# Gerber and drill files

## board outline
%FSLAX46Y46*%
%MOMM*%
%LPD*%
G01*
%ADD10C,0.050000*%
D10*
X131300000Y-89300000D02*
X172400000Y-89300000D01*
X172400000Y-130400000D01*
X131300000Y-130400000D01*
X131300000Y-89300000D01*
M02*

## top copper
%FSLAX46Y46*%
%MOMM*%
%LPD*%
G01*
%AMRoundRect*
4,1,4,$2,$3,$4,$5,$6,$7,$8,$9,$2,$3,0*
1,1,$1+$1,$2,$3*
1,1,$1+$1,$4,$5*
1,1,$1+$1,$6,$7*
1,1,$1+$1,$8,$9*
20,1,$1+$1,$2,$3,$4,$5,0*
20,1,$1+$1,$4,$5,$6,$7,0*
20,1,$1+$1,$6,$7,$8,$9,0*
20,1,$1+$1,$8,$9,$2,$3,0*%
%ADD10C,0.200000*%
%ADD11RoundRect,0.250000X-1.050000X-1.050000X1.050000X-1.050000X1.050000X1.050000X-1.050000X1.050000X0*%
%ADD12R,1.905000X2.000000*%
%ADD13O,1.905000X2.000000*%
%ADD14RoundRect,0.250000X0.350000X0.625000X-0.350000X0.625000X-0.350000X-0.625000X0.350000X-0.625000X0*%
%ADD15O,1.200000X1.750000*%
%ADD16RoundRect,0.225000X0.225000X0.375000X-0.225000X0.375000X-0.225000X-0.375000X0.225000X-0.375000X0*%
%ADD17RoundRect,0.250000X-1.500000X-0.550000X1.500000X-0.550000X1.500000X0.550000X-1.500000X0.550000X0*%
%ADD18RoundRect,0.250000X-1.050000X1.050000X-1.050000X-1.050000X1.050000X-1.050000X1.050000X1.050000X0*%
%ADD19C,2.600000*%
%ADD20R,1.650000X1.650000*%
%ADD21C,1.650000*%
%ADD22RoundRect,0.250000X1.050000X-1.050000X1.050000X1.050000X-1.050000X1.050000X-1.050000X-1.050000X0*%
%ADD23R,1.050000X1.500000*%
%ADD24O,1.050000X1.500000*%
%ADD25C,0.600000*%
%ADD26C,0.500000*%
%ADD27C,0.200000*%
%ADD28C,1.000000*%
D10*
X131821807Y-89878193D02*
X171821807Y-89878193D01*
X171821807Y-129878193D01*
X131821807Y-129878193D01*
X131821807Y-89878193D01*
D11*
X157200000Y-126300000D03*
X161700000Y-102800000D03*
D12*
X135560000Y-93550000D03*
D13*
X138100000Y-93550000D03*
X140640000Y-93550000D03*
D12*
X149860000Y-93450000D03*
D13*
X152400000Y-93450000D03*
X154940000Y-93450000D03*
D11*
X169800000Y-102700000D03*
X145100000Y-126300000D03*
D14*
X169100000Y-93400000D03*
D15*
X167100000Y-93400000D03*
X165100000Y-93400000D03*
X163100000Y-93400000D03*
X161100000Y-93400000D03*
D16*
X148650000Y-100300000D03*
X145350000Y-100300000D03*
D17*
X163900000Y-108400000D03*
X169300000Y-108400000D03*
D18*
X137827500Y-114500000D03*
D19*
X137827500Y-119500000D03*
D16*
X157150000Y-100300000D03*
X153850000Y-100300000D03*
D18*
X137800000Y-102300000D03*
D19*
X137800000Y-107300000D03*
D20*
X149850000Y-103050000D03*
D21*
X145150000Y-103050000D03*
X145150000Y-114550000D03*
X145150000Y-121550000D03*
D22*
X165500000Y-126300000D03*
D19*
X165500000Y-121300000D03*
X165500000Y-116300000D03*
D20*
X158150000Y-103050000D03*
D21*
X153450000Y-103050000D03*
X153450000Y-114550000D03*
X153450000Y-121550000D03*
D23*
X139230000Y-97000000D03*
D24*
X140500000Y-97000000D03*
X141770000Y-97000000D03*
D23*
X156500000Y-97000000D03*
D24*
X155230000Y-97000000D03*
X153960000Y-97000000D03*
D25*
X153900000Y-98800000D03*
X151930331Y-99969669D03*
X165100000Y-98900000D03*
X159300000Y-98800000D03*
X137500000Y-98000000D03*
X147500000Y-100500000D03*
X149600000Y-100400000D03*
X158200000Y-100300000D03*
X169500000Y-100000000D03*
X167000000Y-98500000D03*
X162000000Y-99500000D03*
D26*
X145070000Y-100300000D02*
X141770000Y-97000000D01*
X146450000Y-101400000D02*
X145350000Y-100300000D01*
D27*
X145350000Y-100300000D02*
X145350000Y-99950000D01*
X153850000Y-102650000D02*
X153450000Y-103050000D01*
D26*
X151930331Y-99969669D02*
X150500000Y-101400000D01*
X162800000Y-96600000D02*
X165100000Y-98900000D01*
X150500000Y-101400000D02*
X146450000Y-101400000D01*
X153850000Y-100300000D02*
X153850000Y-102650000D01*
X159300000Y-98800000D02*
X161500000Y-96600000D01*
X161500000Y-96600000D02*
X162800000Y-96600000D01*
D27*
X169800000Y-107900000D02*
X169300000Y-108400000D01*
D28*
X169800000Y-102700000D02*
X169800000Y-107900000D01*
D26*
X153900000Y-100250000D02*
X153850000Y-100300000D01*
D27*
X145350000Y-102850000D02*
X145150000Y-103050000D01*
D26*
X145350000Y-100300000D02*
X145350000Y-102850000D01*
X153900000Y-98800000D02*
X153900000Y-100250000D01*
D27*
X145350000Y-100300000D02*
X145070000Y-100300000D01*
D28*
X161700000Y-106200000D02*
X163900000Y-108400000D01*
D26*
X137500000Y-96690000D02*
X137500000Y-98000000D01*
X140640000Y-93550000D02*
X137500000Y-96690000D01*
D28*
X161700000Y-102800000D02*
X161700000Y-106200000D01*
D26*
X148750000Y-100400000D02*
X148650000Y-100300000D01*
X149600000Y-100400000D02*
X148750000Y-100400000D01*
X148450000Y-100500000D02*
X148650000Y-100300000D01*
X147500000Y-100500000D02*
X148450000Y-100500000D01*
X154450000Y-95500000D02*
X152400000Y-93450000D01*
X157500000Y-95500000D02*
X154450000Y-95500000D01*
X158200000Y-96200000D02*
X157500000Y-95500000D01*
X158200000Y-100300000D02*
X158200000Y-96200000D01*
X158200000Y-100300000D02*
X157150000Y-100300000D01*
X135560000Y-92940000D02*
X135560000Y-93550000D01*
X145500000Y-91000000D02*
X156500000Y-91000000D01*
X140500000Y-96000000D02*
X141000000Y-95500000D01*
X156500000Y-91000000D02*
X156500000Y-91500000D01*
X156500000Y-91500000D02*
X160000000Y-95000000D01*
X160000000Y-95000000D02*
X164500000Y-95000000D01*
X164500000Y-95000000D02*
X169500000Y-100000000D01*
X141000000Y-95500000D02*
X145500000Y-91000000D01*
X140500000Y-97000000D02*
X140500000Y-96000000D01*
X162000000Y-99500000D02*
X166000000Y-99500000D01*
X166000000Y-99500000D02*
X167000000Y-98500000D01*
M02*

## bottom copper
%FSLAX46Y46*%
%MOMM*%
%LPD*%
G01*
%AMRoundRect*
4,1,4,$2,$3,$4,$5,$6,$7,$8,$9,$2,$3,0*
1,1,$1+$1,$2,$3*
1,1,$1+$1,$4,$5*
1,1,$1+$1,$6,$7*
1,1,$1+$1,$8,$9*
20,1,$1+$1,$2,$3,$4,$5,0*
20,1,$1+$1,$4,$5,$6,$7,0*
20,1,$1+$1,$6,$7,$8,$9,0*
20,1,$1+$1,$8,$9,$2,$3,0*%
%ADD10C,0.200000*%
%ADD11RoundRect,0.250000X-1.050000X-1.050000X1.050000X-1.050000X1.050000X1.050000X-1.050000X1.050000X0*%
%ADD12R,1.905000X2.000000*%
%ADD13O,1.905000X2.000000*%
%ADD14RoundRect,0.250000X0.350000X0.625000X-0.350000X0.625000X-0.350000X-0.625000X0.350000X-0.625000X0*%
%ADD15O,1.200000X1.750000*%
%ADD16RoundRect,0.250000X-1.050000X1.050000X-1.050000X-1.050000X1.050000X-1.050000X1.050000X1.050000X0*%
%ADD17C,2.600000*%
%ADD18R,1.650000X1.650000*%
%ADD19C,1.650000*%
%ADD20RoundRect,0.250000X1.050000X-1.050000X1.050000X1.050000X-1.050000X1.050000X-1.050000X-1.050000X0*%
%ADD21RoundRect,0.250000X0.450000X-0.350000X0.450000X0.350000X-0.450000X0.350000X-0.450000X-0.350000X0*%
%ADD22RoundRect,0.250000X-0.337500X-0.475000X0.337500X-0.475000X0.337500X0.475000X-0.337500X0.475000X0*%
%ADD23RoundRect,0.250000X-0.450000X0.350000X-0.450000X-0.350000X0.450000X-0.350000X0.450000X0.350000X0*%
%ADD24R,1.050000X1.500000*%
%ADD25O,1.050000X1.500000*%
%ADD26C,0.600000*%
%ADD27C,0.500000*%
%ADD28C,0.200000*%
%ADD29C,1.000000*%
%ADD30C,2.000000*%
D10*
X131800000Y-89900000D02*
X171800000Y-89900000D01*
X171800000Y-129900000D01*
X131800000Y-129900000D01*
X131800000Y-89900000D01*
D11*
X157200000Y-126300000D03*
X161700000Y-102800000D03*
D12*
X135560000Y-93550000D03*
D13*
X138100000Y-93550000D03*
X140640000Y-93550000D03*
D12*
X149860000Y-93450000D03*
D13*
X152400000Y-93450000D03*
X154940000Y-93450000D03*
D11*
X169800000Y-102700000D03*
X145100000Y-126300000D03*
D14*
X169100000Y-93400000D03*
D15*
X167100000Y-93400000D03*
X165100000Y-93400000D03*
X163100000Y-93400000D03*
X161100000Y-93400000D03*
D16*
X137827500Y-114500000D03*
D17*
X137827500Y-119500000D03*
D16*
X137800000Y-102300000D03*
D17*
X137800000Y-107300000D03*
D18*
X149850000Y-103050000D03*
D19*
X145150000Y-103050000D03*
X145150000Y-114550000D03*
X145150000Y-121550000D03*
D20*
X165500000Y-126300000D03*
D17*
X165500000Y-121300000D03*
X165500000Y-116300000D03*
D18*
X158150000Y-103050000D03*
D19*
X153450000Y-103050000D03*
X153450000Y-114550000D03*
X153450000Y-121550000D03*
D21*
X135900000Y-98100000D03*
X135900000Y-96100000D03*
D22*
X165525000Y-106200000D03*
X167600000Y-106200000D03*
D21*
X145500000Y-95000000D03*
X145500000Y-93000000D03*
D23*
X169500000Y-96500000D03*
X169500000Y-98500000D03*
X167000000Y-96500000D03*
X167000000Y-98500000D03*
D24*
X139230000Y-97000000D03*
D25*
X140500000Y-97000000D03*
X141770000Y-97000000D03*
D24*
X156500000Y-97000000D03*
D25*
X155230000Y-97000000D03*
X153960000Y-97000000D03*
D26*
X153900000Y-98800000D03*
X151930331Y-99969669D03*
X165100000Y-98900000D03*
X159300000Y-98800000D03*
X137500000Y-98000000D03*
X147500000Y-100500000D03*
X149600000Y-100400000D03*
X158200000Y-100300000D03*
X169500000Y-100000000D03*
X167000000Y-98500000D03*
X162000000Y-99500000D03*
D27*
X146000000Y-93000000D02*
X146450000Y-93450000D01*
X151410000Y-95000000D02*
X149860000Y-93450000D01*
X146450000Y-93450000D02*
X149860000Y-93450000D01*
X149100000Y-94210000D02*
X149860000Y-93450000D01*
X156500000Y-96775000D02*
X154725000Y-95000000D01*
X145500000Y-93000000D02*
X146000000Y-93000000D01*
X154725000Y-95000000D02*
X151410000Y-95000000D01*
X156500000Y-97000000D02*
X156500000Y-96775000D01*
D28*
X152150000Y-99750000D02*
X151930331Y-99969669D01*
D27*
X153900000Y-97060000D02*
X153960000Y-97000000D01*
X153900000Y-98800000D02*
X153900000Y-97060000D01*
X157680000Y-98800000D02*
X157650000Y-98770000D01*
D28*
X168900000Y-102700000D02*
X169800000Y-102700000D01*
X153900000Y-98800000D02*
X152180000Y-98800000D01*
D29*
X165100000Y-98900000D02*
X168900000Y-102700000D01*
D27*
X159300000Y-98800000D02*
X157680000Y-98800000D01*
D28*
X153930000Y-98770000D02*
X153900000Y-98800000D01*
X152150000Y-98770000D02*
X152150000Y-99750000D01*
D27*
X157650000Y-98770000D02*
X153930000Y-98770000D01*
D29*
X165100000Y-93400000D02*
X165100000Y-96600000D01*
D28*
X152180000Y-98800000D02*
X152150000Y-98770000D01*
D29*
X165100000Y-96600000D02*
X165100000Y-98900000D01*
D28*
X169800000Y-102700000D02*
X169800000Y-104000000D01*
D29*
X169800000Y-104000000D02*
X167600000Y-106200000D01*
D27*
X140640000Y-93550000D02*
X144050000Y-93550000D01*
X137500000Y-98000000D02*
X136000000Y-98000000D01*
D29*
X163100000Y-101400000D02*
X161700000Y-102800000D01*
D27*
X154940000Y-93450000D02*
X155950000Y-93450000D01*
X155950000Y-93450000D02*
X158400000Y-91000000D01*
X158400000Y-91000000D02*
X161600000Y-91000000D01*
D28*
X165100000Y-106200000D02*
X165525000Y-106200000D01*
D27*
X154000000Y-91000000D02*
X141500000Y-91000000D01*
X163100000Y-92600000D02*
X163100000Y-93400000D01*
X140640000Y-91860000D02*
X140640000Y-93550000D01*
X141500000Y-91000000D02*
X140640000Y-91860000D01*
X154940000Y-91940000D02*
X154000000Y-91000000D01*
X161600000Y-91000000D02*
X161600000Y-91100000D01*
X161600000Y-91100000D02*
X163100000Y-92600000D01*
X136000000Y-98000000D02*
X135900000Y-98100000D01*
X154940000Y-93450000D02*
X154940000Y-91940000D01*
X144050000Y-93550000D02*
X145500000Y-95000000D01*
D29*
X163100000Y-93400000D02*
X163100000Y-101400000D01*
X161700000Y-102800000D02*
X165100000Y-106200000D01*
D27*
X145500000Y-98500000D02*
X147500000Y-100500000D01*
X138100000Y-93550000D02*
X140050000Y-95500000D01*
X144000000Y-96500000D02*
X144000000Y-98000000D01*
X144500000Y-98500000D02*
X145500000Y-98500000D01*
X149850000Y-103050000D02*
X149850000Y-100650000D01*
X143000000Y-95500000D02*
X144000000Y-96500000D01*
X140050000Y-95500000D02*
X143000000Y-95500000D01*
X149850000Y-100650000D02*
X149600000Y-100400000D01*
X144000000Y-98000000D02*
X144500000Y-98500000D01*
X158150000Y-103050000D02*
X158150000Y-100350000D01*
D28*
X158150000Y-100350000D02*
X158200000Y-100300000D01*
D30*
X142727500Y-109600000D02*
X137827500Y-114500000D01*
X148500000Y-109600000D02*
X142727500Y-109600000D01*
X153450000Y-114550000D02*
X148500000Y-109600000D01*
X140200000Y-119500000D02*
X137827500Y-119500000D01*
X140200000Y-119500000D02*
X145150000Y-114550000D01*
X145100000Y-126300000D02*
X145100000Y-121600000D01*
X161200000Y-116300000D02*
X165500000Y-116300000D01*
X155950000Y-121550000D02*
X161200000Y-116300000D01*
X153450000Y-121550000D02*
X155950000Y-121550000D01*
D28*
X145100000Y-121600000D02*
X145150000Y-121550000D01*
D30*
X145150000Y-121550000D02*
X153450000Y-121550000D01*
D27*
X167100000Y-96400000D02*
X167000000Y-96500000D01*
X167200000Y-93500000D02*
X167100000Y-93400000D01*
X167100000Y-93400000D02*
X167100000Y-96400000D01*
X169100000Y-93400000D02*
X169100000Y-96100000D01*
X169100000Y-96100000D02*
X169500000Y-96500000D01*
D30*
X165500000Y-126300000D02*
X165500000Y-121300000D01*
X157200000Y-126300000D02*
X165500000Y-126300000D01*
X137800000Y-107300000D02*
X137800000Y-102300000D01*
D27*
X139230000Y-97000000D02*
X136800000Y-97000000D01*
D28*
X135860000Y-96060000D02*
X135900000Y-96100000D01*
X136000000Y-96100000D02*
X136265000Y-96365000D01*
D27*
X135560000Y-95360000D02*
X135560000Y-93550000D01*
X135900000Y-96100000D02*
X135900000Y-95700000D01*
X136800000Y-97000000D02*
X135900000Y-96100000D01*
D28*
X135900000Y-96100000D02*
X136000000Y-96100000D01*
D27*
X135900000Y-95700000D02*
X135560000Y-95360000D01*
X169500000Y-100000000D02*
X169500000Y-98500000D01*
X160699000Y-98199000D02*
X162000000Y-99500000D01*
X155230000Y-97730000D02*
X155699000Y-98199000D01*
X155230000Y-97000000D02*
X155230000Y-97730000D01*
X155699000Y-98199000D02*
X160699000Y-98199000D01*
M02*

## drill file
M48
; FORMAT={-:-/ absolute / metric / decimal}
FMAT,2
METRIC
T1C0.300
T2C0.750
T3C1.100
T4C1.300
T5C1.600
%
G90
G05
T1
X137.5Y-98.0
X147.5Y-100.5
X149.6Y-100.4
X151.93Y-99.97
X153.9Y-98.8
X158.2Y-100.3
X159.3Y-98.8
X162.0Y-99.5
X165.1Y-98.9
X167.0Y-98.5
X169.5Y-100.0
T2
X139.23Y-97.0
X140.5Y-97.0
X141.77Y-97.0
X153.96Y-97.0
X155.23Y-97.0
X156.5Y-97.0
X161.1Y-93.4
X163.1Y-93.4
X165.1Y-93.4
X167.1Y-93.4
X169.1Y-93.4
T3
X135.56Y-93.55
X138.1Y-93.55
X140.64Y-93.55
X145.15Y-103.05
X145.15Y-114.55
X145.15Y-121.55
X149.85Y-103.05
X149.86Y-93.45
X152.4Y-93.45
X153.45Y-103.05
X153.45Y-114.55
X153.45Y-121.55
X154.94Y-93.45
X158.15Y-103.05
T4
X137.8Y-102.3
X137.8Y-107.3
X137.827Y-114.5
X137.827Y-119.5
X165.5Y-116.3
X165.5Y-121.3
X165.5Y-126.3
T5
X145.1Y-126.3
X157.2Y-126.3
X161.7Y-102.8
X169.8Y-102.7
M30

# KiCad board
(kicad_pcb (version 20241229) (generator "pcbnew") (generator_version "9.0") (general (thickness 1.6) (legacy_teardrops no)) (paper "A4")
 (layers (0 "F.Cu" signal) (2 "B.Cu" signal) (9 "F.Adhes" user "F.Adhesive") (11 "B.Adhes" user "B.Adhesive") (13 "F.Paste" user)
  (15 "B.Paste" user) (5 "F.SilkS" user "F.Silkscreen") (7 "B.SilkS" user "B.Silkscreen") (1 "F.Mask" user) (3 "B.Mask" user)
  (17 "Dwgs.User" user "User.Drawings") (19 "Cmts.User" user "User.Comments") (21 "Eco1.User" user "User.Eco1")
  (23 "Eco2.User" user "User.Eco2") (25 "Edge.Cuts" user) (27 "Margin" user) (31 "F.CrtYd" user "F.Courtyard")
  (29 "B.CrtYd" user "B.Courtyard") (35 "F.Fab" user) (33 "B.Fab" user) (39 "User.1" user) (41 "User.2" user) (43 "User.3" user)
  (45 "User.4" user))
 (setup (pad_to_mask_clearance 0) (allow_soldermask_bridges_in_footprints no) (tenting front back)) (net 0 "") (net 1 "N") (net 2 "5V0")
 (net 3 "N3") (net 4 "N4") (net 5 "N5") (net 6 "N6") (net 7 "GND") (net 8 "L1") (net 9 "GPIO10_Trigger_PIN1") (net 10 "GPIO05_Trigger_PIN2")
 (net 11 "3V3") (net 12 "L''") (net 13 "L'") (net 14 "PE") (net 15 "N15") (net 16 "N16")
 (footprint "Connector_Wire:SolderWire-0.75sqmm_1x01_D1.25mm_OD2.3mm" (layer "F.Cu") (at 157.2 126.3)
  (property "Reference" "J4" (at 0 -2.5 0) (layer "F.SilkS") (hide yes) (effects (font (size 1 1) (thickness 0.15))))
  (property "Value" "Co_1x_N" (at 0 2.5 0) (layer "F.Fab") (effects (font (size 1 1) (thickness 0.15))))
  (pad "1" thru_hole roundrect (at 0 0) (size 2.6 2.6) (drill 1.6) (layers "*.Cu" "*.Mask") (remove_unused_layers no)
   (roundrect_rratio 0.096154) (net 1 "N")))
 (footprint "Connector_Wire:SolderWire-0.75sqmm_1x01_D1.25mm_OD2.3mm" (layer "F.Cu") (at 161.7 102.8)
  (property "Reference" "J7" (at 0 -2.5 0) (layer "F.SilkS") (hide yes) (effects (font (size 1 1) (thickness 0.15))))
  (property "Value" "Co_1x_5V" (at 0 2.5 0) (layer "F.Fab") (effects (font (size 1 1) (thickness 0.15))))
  (pad "1" thru_hole roundrect (at 0 0) (size 2.6 2.6) (drill 1.6) (layers "*.Cu" "*.Mask") (remove_unused_layers no)
   (roundrect_rratio 0.096154) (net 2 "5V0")))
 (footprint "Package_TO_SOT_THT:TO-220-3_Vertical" (layer "F.Cu") (at 135.56 93.55)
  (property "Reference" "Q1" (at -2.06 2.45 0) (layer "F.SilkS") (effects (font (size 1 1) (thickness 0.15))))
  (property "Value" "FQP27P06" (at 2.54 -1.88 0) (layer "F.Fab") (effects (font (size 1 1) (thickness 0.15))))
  (pad "1" thru_hole rect (at 0 0) (size 1.905 2) (drill 1.1) (layers "*.Cu" "*.Mask") (remove_unused_layers no) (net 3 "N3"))
  (pad "2" thru_hole oval (at 2.54 0) (size 1.905 2) (drill 1.1) (layers "*.Cu" "*.Mask") (remove_unused_layers no) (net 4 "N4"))
  (pad "3" thru_hole oval (at 5.08 0) (size 1.905 2) (drill 1.1) (layers "*.Cu" "*.Mask") (remove_unused_layers no) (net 2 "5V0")))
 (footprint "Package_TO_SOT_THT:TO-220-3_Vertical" (layer "F.Cu") (at 149.86 93.45)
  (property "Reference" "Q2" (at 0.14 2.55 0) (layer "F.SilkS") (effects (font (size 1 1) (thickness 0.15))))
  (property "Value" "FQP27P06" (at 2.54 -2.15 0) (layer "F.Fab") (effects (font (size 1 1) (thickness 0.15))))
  (pad "1" thru_hole rect (at 0 0) (size 1.905 2) (drill 1.1) (layers "*.Cu" "*.Mask") (remove_unused_layers no) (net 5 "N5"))
  (pad "2" thru_hole oval (at 2.54 0) (size 1.905 2) (drill 1.1) (layers "*.Cu" "*.Mask") (remove_unused_layers no) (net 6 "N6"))
  (pad "3" thru_hole oval (at 5.08 0) (size 1.905 2) (drill 1.1) (layers "*.Cu" "*.Mask") (remove_unused_layers no) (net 2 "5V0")))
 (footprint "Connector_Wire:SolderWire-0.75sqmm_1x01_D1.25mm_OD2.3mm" (layer "F.Cu") (at 169.8 102.7)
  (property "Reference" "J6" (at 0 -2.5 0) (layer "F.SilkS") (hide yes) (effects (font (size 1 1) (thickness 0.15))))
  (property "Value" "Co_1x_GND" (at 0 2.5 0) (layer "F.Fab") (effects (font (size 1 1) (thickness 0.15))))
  (pad "1" thru_hole roundrect (at 0 0) (size 2.6 2.6) (drill 1.6) (layers "*.Cu" "*.Mask") (remove_unused_layers no)
   (roundrect_rratio 0.096154) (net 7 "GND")))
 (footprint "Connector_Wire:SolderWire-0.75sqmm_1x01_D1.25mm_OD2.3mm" (layer "F.Cu") (at 145.1 126.3)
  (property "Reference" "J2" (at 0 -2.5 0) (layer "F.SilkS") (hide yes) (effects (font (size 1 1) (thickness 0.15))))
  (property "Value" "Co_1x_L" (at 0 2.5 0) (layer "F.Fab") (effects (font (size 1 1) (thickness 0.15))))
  (pad "1" thru_hole roundrect (at 0 0) (size 2.6 2.6) (drill 1.6) (layers "*.Cu" "*.Mask") (remove_unused_layers no)
   (roundrect_rratio 0.096154) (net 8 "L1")))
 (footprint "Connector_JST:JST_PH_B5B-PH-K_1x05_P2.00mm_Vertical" (layer "F.Cu") (at 169.1 93.4 180)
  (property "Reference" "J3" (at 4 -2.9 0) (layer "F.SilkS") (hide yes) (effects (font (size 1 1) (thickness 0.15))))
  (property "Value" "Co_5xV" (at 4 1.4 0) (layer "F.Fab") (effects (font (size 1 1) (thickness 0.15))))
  (pad "1" thru_hole roundrect (at 0 0 180) (size 1.2 1.75) (drill 0.75) (layers "*.Cu" "*.Mask") (remove_unused_layers no)
   (roundrect_rratio 0.208333) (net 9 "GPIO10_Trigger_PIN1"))
  (pad "2" thru_hole oval (at 2 0 180) (size 1.2 1.75) (drill 0.75) (layers "*.Cu" "*.Mask") (remove_unused_layers no)
   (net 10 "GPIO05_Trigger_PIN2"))
  (pad "3" thru_hole oval (at 4 0 180) (size 1.2 1.75) (drill 0.75) (layers "*.Cu" "*.Mask") (remove_unused_layers no) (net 7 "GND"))
  (pad "4" thru_hole oval (at 6 0 180) (size 1.2 1.75) (drill 0.75) (layers "*.Cu" "*.Mask") (remove_unused_layers no) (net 2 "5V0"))
  (pad "5" thru_hole oval (at 8 0 180) (size 1.2 1.75) (drill 0.75) (layers "*.Cu" "*.Mask") (remove_unused_layers no) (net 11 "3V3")))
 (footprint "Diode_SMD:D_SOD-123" (layer "F.Cu") (at 147 100.3 180)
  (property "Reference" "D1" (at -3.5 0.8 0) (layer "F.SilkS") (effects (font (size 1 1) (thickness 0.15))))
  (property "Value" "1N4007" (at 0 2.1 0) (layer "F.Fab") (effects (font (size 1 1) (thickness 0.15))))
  (pad "1" smd roundrect (at -1.65 0 180) (size 0.9 1.2) (layers "F.Cu" "F.Mask" "F.Paste") (roundrect_rratio 0.25) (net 4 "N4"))
  (pad "2" smd roundrect (at 1.65 0 180) (size 0.9 1.2) (layers "F.Cu" "F.Mask" "F.Paste") (roundrect_rratio 0.25) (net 7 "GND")))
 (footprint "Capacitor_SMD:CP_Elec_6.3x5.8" (layer "F.Cu") (at 166.6 108.4)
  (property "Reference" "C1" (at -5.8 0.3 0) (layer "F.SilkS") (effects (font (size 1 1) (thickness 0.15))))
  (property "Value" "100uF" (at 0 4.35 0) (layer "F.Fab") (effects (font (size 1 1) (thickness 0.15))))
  (pad "1" smd roundrect (at -2.7 0) (size 3.5 1.6) (layers "F.Cu" "F.Mask" "F.Paste") (roundrect_rratio 0.15625) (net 2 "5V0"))
  (pad "2" smd roundrect (at 2.7 0) (size 3.5 1.6) (layers "F.Cu" "F.Mask" "F.Paste") (roundrect_rratio 0.15625) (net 7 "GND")))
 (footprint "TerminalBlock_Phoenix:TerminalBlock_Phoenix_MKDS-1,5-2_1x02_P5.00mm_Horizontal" (layer "F.Cu") (at 137.8275 114.5 -90)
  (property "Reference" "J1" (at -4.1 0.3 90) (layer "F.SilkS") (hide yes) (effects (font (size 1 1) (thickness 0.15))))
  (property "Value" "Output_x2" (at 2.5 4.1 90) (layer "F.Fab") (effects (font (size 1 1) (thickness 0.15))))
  (pad "1" thru_hole roundrect (at 0 0 270) (size 2.6 2.6) (drill 1.3) (layers "*.Cu" "*.Mask") (remove_unused_layers no)
   (roundrect_rratio 0.096154) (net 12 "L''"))
  (pad "2" thru_hole circle (at 5 0 270) (size 2.6 2.6) (drill 1.3) (layers "*.Cu" "*.Mask") (remove_unused_layers no) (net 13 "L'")))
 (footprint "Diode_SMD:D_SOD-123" (layer "F.Cu") (at 155.5 100.3 180)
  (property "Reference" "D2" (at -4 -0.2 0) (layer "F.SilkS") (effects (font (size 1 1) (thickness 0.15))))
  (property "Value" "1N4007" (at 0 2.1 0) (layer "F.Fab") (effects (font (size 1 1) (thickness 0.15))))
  (pad "1" smd roundrect (at -1.65 0 180) (size 0.9 1.2) (layers "F.Cu" "F.Mask" "F.Paste") (roundrect_rratio 0.25) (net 6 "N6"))
  (pad "2" smd roundrect (at 1.65 0 180) (size 0.9 1.2) (layers "F.Cu" "F.Mask" "F.Paste") (roundrect_rratio 0.25) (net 7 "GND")))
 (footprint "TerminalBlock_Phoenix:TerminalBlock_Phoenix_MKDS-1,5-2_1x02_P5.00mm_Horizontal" (layer "F.Cu") (at 137.8 102.3 -90)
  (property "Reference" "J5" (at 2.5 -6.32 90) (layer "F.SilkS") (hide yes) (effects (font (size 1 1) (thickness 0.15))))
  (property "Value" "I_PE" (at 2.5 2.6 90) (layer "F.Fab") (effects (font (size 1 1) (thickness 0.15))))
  (pad "1" thru_hole roundrect (at 0 0 270) (size 2.6 2.6) (drill 1.3) (layers "*.Cu" "*.Mask") (remove_unused_layers no)
   (roundrect_rratio 0.096154) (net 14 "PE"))
  (pad "2" thru_hole circle (at 5 0 270) (size 2.6 2.6) (drill 1.3) (layers "*.Cu" "*.Mask") (remove_unused_layers no) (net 14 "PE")))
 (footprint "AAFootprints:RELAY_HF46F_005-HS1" (layer "F.Cu") (at 147.5 112.25 -90)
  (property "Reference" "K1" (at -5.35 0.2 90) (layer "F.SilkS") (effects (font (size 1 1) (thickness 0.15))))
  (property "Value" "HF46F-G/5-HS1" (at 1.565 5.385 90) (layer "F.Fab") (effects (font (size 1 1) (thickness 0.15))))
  (pad "1" thru_hole rect (at -9.2 -2.35 270) (size 1.65 1.65) (drill 1.1) (layers "*.Cu" "*.Mask") (remove_unused_layers no) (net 4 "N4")
   (solder_mask_margin 0.102))
  (pad "2" thru_hole circle (at -9.2 2.35 270) (size 1.65 1.65) (drill 1.1) (layers "*.Cu" "*.Mask") (remove_unused_layers no) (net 7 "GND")
   (solder_mask_margin 0.102))
  (pad "3" thru_hole circle (at 2.3 2.35 270) (size 1.65 1.65) (drill 1.1) (layers "*.Cu" "*.Mask") (remove_unused_layers no) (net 13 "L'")
   (solder_mask_margin 0.102))
  (pad "4" thru_hole circle (at 9.3 2.35 270) (size 1.65 1.65) (drill 1.1) (layers "*.Cu" "*.Mask") (remove_unused_layers no) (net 8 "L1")
   (solder_mask_margin 0.102)))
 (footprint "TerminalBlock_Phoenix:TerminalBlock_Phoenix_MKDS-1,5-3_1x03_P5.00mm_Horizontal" (layer "F.Cu") (at 165.5 126.3 90)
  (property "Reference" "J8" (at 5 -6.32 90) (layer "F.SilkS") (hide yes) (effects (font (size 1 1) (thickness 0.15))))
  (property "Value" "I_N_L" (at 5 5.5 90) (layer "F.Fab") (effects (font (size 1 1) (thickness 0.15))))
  (pad "1" thru_hole roundrect (at 0 0 90) (size 2.6 2.6) (drill 1.3) (layers "*.Cu" "*.Mask") (remove_unused_layers no)
   (roundrect_rratio 0.096154) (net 1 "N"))
  (pad "2" thru_hole circle (at 5 0 90) (size 2.6 2.6) (drill 1.3) (layers "*.Cu" "*.Mask") (remove_unused_layers no) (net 1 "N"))
  (pad "3" thru_hole circle (at 10 0 90) (size 2.6 2.6) (drill 1.3) (layers "*.Cu" "*.Mask") (remove_unused_layers no) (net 8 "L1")))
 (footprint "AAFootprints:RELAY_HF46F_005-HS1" (layer "F.Cu") (at 155.8 112.25 -90)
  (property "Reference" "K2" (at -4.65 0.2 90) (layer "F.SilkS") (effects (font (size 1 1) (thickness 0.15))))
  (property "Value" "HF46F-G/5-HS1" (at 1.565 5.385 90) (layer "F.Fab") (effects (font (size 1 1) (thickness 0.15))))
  (pad "1" thru_hole rect (at -9.2 -2.35 270) (size 1.65 1.65) (drill 1.1) (layers "*.Cu" "*.Mask") (remove_unused_layers no) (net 6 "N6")
   (solder_mask_margin 0.102))
  (pad "2" thru_hole circle (at -9.2 2.35 270) (size 1.65 1.65) (drill 1.1) (layers "*.Cu" "*.Mask") (remove_unused_layers no) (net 7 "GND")
   (solder_mask_margin 0.102))
  (pad "3" thru_hole circle (at 2.3 2.35 270) (size 1.65 1.65) (drill 1.1) (layers "*.Cu" "*.Mask") (remove_unused_layers no) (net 12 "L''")
   (solder_mask_margin 0.102))
  (pad "4" thru_hole circle (at 9.3 2.35 270) (size 1.65 1.65) (drill 1.1) (layers "*.Cu" "*.Mask") (remove_unused_layers no) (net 8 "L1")
   (solder_mask_margin 0.102)))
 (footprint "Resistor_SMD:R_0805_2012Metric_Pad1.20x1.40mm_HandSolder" (layer "B.Cu") (at 135.9 97.1 90)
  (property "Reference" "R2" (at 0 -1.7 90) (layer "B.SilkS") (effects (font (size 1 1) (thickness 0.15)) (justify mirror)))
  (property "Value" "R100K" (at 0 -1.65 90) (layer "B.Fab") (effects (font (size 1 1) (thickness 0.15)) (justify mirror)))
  (pad "1" smd roundrect (at -1 0 90) (size 1.2 1.4) (layers "B.Cu" "B.Mask" "B.Paste") (roundrect_rratio 0.208333) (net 2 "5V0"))
  (pad "2" smd roundrect (at 1 0 90) (size 1.2 1.4) (layers "B.Cu" "B.Mask" "B.Paste") (roundrect_rratio 0.208333) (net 3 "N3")))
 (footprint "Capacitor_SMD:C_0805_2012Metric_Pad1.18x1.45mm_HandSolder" (layer "B.Cu") (at 166.5625 106.2)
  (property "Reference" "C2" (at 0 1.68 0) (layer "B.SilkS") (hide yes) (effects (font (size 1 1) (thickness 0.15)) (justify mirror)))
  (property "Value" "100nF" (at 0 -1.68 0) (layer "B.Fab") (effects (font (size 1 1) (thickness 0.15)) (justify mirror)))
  (pad "1" smd roundrect (at -1.0375 0) (size 1.175 1.45) (layers "B.Cu" "B.Mask" "B.Paste") (roundrect_rratio 0.212766) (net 2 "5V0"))
  (pad "2" smd roundrect (at 1.0375 0) (size 1.175 1.45) (layers "B.Cu" "B.Mask" "B.Paste") (roundrect_rratio 0.212766) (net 7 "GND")))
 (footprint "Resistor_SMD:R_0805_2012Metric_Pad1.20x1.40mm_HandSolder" (layer "B.Cu") (at 145.5 94 90)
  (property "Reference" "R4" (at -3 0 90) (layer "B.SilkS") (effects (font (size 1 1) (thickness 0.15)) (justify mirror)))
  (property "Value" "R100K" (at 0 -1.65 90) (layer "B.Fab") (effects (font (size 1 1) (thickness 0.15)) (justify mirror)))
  (pad "1" smd roundrect (at -1 0 90) (size 1.2 1.4) (layers "B.Cu" "B.Mask" "B.Paste") (roundrect_rratio 0.208333) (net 2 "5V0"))
  (pad "2" smd roundrect (at 1 0 90) (size 1.2 1.4) (layers "B.Cu" "B.Mask" "B.Paste") (roundrect_rratio 0.208333) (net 5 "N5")))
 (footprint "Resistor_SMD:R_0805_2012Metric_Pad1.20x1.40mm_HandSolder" (layer "B.Cu") (at 169.5 97.5 -90)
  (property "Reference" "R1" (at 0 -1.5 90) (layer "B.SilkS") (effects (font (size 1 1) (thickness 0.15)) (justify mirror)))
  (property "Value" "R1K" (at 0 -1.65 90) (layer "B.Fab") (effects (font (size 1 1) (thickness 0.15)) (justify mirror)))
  (pad "1" smd roundrect (at -1 0 270) (size 1.2 1.4) (layers "B.Cu" "B.Mask" "B.Paste") (roundrect_rratio 0.208333)
   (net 9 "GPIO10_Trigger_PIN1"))
  (pad "2" smd roundrect (at 1 0 270) (size 1.2 1.4) (layers "B.Cu" "B.Mask" "B.Paste") (roundrect_rratio 0.208333) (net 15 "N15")))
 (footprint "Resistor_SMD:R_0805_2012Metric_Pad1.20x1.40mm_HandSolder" (layer "B.Cu") (at 167 97.5 -90)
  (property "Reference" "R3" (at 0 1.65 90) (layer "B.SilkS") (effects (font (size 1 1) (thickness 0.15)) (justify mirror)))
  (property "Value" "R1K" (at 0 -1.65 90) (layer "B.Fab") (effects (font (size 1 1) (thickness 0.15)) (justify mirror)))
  (pad "1" smd roundrect (at -1 0 270) (size 1.2 1.4) (layers "B.Cu" "B.Mask" "B.Paste") (roundrect_rratio 0.208333)
   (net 10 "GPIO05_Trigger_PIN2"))
  (pad "2" smd roundrect (at 1 0 270) (size 1.2 1.4) (layers "B.Cu" "B.Mask" "B.Paste") (roundrect_rratio 0.208333) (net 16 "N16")))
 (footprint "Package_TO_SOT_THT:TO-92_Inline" (layer "B.Cu") (at 139.23 97)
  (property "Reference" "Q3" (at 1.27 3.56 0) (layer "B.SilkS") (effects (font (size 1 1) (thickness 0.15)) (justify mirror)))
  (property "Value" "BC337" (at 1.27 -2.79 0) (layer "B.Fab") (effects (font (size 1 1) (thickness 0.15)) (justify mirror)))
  (pad "1" thru_hole rect (at 0 0) (size 1.05 1.5) (drill 0.75) (layers "*.Cu" "*.Mask") (remove_unused_layers no) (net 3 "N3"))
  (pad "2" thru_hole oval (at 1.27 0) (size 1.05 1.5) (drill 0.75) (layers "*.Cu" "*.Mask") (remove_unused_layers no) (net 15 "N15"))
  (pad "3" thru_hole oval (at 2.54 0) (size 1.05 1.5) (drill 0.75) (layers "*.Cu" "*.Mask") (remove_unused_layers no) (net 7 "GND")))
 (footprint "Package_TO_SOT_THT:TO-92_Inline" (layer "B.Cu") (at 156.5 97 180)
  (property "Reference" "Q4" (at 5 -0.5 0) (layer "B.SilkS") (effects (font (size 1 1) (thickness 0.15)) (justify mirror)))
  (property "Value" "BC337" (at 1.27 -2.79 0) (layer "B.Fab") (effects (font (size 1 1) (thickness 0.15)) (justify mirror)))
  (pad "1" thru_hole rect (at 0 0 180) (size 1.05 1.5) (drill 0.75) (layers "*.Cu" "*.Mask") (remove_unused_layers no) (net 5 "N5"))
  (pad "2" thru_hole oval (at 1.27 0 180) (size 1.05 1.5) (drill 0.75) (layers "*.Cu" "*.Mask") (remove_unused_layers no) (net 16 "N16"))
  (pad "3" thru_hole oval (at 2.54 0 180) (size 1.05 1.5) (drill 0.75) (layers "*.Cu" "*.Mask") (remove_unused_layers no) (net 7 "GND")))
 (gr_rect (start 131.821807 89.878193) (end 171.821807 129.878193) (stroke (width 0.2) (type solid)) (fill no) (layer "F.Cu"))
 (gr_rect (start 131.8 89.9) (end 171.8 129.9) (stroke (width 0.2) (type default)) (fill no) (layer "B.Cu"))
 (gr_rect (start 131.3 89.3) (end 172.4 130.4) (stroke (width 0.05) (type solid)) (fill no) (layer "Edge.Cuts"))
 (segment (start 146 93) (end 146.45 93.45) (width 0.5) (layer "B.Cu") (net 5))
 (segment (start 151.41 95) (end 149.86 93.45) (width 0.5) (layer "B.Cu") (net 5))
 (segment (start 146.45 93.45) (end 149.86 93.45) (width 0.5) (layer "B.Cu") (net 5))
 (segment (start 149.1 94.21) (end 149.86 93.45) (width 0.5) (layer "B.Cu") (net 5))
 (segment (start 156.5 96.775) (end 154.725 95) (width 0.5) (layer "B.Cu") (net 5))
 (segment (start 145.5 93) (end 146 93) (width 0.5) (layer "B.Cu") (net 5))
 (segment (start 154.725 95) (end 151.41 95) (width 0.5) (layer "B.Cu") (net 5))
 (segment (start 156.5 97) (end 156.5 96.775) (width 0.5) (layer "B.Cu") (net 5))
 (segment (start 145.07 100.3) (end 141.77 97) (width 0.5) (layer "F.Cu") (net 7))
 (segment (start 146.45 101.4) (end 145.35 100.3) (width 0.5) (layer "F.Cu") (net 7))
 (segment (start 145.35 100.3) (end 145.35 99.95) (width 0.2) (layer "F.Cu") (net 7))
 (segment (start 153.85 102.65) (end 153.45 103.05) (width 0.2) (layer "F.Cu") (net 7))
 (segment (start 151.930331 99.969669) (end 150.5 101.4) (width 0.5) (layer "F.Cu") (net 7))
 (segment (start 162.8 96.6) (end 165.1 98.9) (width 0.5) (layer "F.Cu") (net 7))
 (segment (start 150.5 101.4) (end 146.45 101.4) (width 0.5) (layer "F.Cu") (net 7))
 (segment (start 153.85 100.3) (end 153.85 102.65) (width 0.5) (layer "F.Cu") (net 7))
 (segment (start 159.3 98.8) (end 161.5 96.6) (width 0.5) (layer "F.Cu") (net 7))
 (segment (start 161.5 96.6) (end 162.8 96.6) (width 0.5) (layer "F.Cu") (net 7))
 (segment (start 169.8 107.9) (end 169.3 108.4) (width 0.2) (layer "F.Cu") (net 7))
 (segment (start 169.8 102.7) (end 169.8 107.9) (width 1) (layer "F.Cu") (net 7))
 (segment (start 153.9 100.25) (end 153.85 100.3) (width 0.5) (layer "F.Cu") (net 7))
 (segment (start 145.35 102.85) (end 145.15 103.05) (width 0.2) (layer "F.Cu") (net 7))
 (segment (start 145.35 100.3) (end 145.35 102.85) (width 0.5) (layer "F.Cu") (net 7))
 (segment (start 153.9 98.8) (end 153.9 100.25) (width 0.5) (layer "F.Cu") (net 7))
 (segment (start 145.35 100.3) (end 145.07 100.3) (width 0.2) (layer "F.Cu") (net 7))
 (via (at 153.9 98.8) (size 0.6) (drill 0.3) (layers "F.Cu" "B.Cu") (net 7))
 (via (at 151.930331 99.969669) (size 0.6) (drill 0.3) (layers "F.Cu" "B.Cu") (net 7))
 (via (at 165.1 98.9) (size 0.6) (drill 0.3) (layers "F.Cu" "B.Cu") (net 7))
 (via (at 159.3 98.8) (size 0.6) (drill 0.3) (layers "F.Cu" "B.Cu") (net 7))
 (segment (start 152.15 99.75) (end 151.930331 99.969669) (width 0.2) (layer "B.Cu") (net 7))
 (segment (start 153.9 97.06) (end 153.96 97) (width 0.5) (layer "B.Cu") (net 7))
 (segment (start 153.9 98.8) (end 153.9 97.06) (width 0.5) (layer "B.Cu") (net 7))
 (segment (start 157.68 98.8) (end 157.65 98.77) (width 0.5) (layer "B.Cu") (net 7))
 (segment (start 168.9 102.7) (end 169.8 102.7) (width 0.2) (layer "B.Cu") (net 7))
 (segment (start 153.9 98.8) (end 152.18 98.8) (width 0.2) (layer "B.Cu") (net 7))
 (segment (start 165.1 98.9) (end 168.9 102.7) (width 1) (layer "B.Cu") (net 7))
 (segment (start 159.3 98.8) (end 157.68 98.8) (width 0.5) (layer "B.Cu") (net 7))
 (segment (start 153.93 98.77) (end 153.9 98.8) (width 0.2) (layer "B.Cu") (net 7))
 (segment (start 152.15 98.77) (end 152.15 99.75) (width 0.2) (layer "B.Cu") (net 7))
 (segment (start 157.65 98.77) (end 153.93 98.77) (width 0.5) (layer "B.Cu") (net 7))
 (segment (start 165.1 93.4) (end 165.1 96.6) (width 1) (layer "B.Cu") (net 7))
 (segment (start 152.18 98.8) (end 152.15 98.77) (width 0.2) (layer "B.Cu") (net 7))
 (segment (start 165.1 96.6) (end 165.1 98.9) (width 1) (layer "B.Cu") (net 7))
 (segment (start 169.8 102.7) (end 169.8 104) (width 0.2) (layer "B.Cu") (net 7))
 (segment (start 169.8 104) (end 167.6 106.2) (width 1) (layer "B.Cu") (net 7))
 (segment (start 161.7 106.2) (end 163.9 108.4) (width 1) (layer "F.Cu") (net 2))
 (segment (start 137.5 96.69) (end 137.5 98) (width 0.5) (layer "F.Cu") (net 2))
 (segment (start 140.64 93.55) (end 137.5 96.69) (width 0.5) (layer "F.Cu") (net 2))
 (segment (start 161.7 102.8) (end 161.7 106.2) (width 1) (layer "F.Cu") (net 2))
 (via (at 137.5 98) (size 0.6) (drill 0.3) (layers "F.Cu" "B.Cu") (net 2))
 (segment (start 140.64 93.55) (end 144.05 93.55) (width 0.5) (layer "B.Cu") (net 2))
 (segment (start 137.5 98) (end 136 98) (width 0.5) (layer "B.Cu") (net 2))
 (segment (start 163.1 101.4) (end 161.7 102.8) (width 1) (layer "B.Cu") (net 2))
 (segment (start 154.94 93.45) (end 155.95 93.45) (width 0.5) (layer "B.Cu") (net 2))
 (segment (start 155.95 93.45) (end 158.4 91) (width 0.5) (layer "B.Cu") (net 2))
 (segment (start 158.4 91) (end 161.6 91) (width 0.5) (layer "B.Cu") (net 2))
 (segment (start 165.1 106.2) (end 165.525 106.2) (width 0.2) (layer "B.Cu") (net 2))
 (segment (start 154 91) (end 141.5 91) (width 0.5) (layer "B.Cu") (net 2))
 (segment (start 163.1 92.6) (end 163.1 93.4) (width 0.5) (layer "B.Cu") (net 2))
 (segment (start 140.64 91.86) (end 140.64 93.55) (width 0.5) (layer "B.Cu") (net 2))
 (segment (start 141.5 91) (end 140.64 91.86) (width 0.5) (layer "B.Cu") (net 2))
 (segment (start 154.94 91.94) (end 154 91) (width 0.5) (layer "B.Cu") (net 2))
 (segment (start 161.6 91) (end 161.6 91.1) (width 0.5) (layer "B.Cu") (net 2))
 (segment (start 161.6 91.1) (end 163.1 92.6) (width 0.5) (layer "B.Cu") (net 2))
 (segment (start 136 98) (end 135.9 98.1) (width 0.5) (layer "B.Cu") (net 2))
 (segment (start 154.94 93.45) (end 154.94 91.94) (width 0.5) (layer "B.Cu") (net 2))
 (segment (start 144.05 93.55) (end 145.5 95) (width 0.5) (layer "B.Cu") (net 2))
 (segment (start 163.1 93.4) (end 163.1 101.4) (width 1) (layer "B.Cu") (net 2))
 (segment (start 161.7 102.8) (end 165.1 106.2) (width 1) (layer "B.Cu") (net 2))
 (segment (start 148.75 100.4) (end 148.65 100.3) (width 0.5) (layer "F.Cu") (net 4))
 (segment (start 149.6 100.4) (end 148.75 100.4) (width 0.5) (layer "F.Cu") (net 4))
 (segment (start 148.45 100.5) (end 148.65 100.3) (width 0.5) (layer "F.Cu") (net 4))
 (segment (start 147.5 100.5) (end 148.45 100.5) (width 0.5) (layer "F.Cu") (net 4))
 (via (at 147.5 100.5) (size 0.6) (drill 0.3) (layers "F.Cu" "B.Cu") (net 4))
 (via (at 149.6 100.4) (size 0.6) (drill 0.3) (layers "F.Cu" "B.Cu") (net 4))
 (segment (start 145.5 98.5) (end 147.5 100.5) (width 0.5) (layer "B.Cu") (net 4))
 (segment (start 138.1 93.55) (end 140.05 95.5) (width 0.5) (layer "B.Cu") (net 4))
 (segment (start 144 96.5) (end 144 98) (width 0.5) (layer "B.Cu") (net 4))
 (segment (start 144.5 98.5) (end 145.5 98.5) (width 0.5) (layer "B.Cu") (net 4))
 (segment (start 149.85 103.05) (end 149.85 100.65) (width 0.5) (layer "B.Cu") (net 4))
 (segment (start 143 95.5) (end 144 96.5) (width 0.5) (layer "B.Cu") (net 4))
 (segment (start 140.05 95.5) (end 143 95.5) (width 0.5) (layer "B.Cu") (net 4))
 (segment (start 149.85 100.65) (end 149.6 100.4) (width 0.5) (layer "B.Cu") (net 4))
 (segment (start 144 98) (end 144.5 98.5) (width 0.5) (layer "B.Cu") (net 4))
 (segment (start 154.45 95.5) (end 152.4 93.45) (width 0.5) (layer "F.Cu") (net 6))
 (segment (start 157.5 95.5) (end 154.45 95.5) (width 0.5) (layer "F.Cu") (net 6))
 (segment (start 158.2 96.2) (end 157.5 95.5) (width 0.5) (layer "F.Cu") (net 6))
 (segment (start 158.2 100.3) (end 158.2 96.2) (width 0.5) (layer "F.Cu") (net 6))
 (segment (start 158.2 100.3) (end 157.15 100.3) (width 0.5) (layer "F.Cu") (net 6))
 (via (at 158.2 100.3) (size 0.6) (drill 0.3) (layers "F.Cu" "B.Cu") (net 6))
 (segment (start 158.15 103.05) (end 158.15 100.35) (width 0.5) (layer "B.Cu") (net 6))
 (segment (start 158.15 100.35) (end 158.2 100.3) (width 0.2) (layer "B.Cu") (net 6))
 (segment (start 142.7275 109.6) (end 137.8275 114.5) (width 2) (layer "B.Cu") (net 12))
 (segment (start 148.5 109.6) (end 142.7275 109.6) (width 2) (layer "B.Cu") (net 12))
 (segment (start 153.45 114.55) (end 148.5 109.6) (width 2) (layer "B.Cu") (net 12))
 (segment (start 140.2 119.5) (end 137.8275 119.5) (width 2) (layer "B.Cu") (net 13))
 (segment (start 140.2 119.5) (end 145.15 114.55) (width 2) (layer "B.Cu") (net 13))
 (segment (start 145.1 126.3) (end 145.1 121.6) (width 2) (layer "B.Cu") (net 8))
 (segment (start 161.2 116.3) (end 165.5 116.3) (width 2) (layer "B.Cu") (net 8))
 (segment (start 155.95 121.55) (end 161.2 116.3) (width 2) (layer "B.Cu") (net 8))
 (segment (start 153.45 121.55) (end 155.95 121.55) (width 2) (layer "B.Cu") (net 8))
 (segment (start 145.1 121.6) (end 145.15 121.55) (width 0.2) (layer "B.Cu") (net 8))
 (segment (start 145.15 121.55) (end 153.45 121.55) (width 2) (layer "B.Cu") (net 8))
 (segment (start 167.1 96.4) (end 167 96.5) (width 0.5) (layer "B.Cu") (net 10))
 (segment (start 167.2 93.5) (end 167.1 93.4) (width 0.5) (layer "B.Cu") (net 10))
 (segment (start 167.1 93.4) (end 167.1 96.4) (width 0.5) (layer "B.Cu") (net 10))
 (segment (start 169.1 93.4) (end 169.1 96.1) (width 0.5) (layer "B.Cu") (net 9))
 (segment (start 169.1 96.1) (end 169.5 96.5) (width 0.5) (layer "B.Cu") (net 9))
 (segment (start 165.5 126.3) (end 165.5 121.3) (width 2) (layer "B.Cu") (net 1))
 (segment (start 157.2 126.3) (end 165.5 126.3) (width 2) (layer "B.Cu") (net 1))
 (segment (start 137.8 107.3) (end 137.8 102.3) (width 2) (layer "B.Cu") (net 14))
 (segment (start 135.56 92.94) (end 135.56 93.55) (width 0.5) (layer "F.Cu") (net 3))
 (segment (start 139.23 97) (end 136.8 97) (width 0.5) (layer "B.Cu") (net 3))
 (segment (start 135.86 96.06) (end 135.9 96.1) (width 0.2) (layer "B.Cu") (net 3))
 (segment (start 136 96.1) (end 136.265 96.365) (width 0.2) (layer "B.Cu") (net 3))
 (segment (start 135.56 95.36) (end 135.56 93.55) (width 0.5) (layer "B.Cu") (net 3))
 (segment (start 135.9 96.1) (end 135.9 95.7) (width 0.5) (layer "B.Cu") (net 3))
 (segment (start 136.8 97) (end 135.9 96.1) (width 0.5) (layer "B.Cu") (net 3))
 (segment (start 135.9 96.1) (end 136 96.1) (width 0.2) (layer "B.Cu") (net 3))
 (segment (start 135.9 95.7) (end 135.56 95.36) (width 0.5) (layer "B.Cu") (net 3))
 (segment (start 145.5 91) (end 156.5 91) (width 0.5) (layers "F.Cu" "F.Mask") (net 15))
 (segment (start 140.5 96) (end 141 95.5) (width 0.5) (layer "F.Cu") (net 15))
 (segment (start 156.5 91) (end 156.5 91.5) (width 0.5) (layer "F.Cu") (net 15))
 (segment (start 156.5 91.5) (end 160 95) (width 0.5) (layer "F.Cu") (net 15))
 (segment (start 160 95) (end 164.5 95) (width 0.5) (layer "F.Cu") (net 15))
 (segment (start 164.5 95) (end 169.5 100) (width 0.5) (layer "F.Cu") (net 15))
 (segment (start 141 95.5) (end 145.5 91) (width 0.5) (layer "F.Cu") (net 15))
 (segment (start 140.5 97) (end 140.5 96) (width 0.5) (layer "F.Cu") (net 15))
 (via (at 169.5 100) (size 0.6) (drill 0.3) (layers "F.Cu" "B.Cu") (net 15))
 (segment (start 169.5 100) (end 169.5 98.5) (width 0.5) (layer "B.Cu") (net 15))
 (segment (start 162 99.5) (end 166 99.5) (width 0.5) (layer "F.Cu") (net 16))
 (segment (start 166 99.5) (end 167 98.5) (width 0.5) (layer "F.Cu") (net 16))
 (via (at 167 98.5) (size 0.6) (drill 0.3) (layers "F.Cu" "B.Cu") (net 16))
 (via (at 162 99.5) (size 0.6) (drill 0.3) (layers "F.Cu" "B.Cu") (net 16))
 (segment (start 160.699 98.199) (end 162 99.5) (width 0.5) (layer "B.Cu") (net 16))
 (segment (start 155.23 97.73) (end 155.699 98.199) (width 0.5) (layer "B.Cu") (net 16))
 (segment (start 155.23 97) (end 155.23 97.73) (width 0.5) (layer "B.Cu") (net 16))
 (segment (start 155.699 98.199) (end 160.699 98.199) (width 0.5) (layer "B.Cu") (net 16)))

